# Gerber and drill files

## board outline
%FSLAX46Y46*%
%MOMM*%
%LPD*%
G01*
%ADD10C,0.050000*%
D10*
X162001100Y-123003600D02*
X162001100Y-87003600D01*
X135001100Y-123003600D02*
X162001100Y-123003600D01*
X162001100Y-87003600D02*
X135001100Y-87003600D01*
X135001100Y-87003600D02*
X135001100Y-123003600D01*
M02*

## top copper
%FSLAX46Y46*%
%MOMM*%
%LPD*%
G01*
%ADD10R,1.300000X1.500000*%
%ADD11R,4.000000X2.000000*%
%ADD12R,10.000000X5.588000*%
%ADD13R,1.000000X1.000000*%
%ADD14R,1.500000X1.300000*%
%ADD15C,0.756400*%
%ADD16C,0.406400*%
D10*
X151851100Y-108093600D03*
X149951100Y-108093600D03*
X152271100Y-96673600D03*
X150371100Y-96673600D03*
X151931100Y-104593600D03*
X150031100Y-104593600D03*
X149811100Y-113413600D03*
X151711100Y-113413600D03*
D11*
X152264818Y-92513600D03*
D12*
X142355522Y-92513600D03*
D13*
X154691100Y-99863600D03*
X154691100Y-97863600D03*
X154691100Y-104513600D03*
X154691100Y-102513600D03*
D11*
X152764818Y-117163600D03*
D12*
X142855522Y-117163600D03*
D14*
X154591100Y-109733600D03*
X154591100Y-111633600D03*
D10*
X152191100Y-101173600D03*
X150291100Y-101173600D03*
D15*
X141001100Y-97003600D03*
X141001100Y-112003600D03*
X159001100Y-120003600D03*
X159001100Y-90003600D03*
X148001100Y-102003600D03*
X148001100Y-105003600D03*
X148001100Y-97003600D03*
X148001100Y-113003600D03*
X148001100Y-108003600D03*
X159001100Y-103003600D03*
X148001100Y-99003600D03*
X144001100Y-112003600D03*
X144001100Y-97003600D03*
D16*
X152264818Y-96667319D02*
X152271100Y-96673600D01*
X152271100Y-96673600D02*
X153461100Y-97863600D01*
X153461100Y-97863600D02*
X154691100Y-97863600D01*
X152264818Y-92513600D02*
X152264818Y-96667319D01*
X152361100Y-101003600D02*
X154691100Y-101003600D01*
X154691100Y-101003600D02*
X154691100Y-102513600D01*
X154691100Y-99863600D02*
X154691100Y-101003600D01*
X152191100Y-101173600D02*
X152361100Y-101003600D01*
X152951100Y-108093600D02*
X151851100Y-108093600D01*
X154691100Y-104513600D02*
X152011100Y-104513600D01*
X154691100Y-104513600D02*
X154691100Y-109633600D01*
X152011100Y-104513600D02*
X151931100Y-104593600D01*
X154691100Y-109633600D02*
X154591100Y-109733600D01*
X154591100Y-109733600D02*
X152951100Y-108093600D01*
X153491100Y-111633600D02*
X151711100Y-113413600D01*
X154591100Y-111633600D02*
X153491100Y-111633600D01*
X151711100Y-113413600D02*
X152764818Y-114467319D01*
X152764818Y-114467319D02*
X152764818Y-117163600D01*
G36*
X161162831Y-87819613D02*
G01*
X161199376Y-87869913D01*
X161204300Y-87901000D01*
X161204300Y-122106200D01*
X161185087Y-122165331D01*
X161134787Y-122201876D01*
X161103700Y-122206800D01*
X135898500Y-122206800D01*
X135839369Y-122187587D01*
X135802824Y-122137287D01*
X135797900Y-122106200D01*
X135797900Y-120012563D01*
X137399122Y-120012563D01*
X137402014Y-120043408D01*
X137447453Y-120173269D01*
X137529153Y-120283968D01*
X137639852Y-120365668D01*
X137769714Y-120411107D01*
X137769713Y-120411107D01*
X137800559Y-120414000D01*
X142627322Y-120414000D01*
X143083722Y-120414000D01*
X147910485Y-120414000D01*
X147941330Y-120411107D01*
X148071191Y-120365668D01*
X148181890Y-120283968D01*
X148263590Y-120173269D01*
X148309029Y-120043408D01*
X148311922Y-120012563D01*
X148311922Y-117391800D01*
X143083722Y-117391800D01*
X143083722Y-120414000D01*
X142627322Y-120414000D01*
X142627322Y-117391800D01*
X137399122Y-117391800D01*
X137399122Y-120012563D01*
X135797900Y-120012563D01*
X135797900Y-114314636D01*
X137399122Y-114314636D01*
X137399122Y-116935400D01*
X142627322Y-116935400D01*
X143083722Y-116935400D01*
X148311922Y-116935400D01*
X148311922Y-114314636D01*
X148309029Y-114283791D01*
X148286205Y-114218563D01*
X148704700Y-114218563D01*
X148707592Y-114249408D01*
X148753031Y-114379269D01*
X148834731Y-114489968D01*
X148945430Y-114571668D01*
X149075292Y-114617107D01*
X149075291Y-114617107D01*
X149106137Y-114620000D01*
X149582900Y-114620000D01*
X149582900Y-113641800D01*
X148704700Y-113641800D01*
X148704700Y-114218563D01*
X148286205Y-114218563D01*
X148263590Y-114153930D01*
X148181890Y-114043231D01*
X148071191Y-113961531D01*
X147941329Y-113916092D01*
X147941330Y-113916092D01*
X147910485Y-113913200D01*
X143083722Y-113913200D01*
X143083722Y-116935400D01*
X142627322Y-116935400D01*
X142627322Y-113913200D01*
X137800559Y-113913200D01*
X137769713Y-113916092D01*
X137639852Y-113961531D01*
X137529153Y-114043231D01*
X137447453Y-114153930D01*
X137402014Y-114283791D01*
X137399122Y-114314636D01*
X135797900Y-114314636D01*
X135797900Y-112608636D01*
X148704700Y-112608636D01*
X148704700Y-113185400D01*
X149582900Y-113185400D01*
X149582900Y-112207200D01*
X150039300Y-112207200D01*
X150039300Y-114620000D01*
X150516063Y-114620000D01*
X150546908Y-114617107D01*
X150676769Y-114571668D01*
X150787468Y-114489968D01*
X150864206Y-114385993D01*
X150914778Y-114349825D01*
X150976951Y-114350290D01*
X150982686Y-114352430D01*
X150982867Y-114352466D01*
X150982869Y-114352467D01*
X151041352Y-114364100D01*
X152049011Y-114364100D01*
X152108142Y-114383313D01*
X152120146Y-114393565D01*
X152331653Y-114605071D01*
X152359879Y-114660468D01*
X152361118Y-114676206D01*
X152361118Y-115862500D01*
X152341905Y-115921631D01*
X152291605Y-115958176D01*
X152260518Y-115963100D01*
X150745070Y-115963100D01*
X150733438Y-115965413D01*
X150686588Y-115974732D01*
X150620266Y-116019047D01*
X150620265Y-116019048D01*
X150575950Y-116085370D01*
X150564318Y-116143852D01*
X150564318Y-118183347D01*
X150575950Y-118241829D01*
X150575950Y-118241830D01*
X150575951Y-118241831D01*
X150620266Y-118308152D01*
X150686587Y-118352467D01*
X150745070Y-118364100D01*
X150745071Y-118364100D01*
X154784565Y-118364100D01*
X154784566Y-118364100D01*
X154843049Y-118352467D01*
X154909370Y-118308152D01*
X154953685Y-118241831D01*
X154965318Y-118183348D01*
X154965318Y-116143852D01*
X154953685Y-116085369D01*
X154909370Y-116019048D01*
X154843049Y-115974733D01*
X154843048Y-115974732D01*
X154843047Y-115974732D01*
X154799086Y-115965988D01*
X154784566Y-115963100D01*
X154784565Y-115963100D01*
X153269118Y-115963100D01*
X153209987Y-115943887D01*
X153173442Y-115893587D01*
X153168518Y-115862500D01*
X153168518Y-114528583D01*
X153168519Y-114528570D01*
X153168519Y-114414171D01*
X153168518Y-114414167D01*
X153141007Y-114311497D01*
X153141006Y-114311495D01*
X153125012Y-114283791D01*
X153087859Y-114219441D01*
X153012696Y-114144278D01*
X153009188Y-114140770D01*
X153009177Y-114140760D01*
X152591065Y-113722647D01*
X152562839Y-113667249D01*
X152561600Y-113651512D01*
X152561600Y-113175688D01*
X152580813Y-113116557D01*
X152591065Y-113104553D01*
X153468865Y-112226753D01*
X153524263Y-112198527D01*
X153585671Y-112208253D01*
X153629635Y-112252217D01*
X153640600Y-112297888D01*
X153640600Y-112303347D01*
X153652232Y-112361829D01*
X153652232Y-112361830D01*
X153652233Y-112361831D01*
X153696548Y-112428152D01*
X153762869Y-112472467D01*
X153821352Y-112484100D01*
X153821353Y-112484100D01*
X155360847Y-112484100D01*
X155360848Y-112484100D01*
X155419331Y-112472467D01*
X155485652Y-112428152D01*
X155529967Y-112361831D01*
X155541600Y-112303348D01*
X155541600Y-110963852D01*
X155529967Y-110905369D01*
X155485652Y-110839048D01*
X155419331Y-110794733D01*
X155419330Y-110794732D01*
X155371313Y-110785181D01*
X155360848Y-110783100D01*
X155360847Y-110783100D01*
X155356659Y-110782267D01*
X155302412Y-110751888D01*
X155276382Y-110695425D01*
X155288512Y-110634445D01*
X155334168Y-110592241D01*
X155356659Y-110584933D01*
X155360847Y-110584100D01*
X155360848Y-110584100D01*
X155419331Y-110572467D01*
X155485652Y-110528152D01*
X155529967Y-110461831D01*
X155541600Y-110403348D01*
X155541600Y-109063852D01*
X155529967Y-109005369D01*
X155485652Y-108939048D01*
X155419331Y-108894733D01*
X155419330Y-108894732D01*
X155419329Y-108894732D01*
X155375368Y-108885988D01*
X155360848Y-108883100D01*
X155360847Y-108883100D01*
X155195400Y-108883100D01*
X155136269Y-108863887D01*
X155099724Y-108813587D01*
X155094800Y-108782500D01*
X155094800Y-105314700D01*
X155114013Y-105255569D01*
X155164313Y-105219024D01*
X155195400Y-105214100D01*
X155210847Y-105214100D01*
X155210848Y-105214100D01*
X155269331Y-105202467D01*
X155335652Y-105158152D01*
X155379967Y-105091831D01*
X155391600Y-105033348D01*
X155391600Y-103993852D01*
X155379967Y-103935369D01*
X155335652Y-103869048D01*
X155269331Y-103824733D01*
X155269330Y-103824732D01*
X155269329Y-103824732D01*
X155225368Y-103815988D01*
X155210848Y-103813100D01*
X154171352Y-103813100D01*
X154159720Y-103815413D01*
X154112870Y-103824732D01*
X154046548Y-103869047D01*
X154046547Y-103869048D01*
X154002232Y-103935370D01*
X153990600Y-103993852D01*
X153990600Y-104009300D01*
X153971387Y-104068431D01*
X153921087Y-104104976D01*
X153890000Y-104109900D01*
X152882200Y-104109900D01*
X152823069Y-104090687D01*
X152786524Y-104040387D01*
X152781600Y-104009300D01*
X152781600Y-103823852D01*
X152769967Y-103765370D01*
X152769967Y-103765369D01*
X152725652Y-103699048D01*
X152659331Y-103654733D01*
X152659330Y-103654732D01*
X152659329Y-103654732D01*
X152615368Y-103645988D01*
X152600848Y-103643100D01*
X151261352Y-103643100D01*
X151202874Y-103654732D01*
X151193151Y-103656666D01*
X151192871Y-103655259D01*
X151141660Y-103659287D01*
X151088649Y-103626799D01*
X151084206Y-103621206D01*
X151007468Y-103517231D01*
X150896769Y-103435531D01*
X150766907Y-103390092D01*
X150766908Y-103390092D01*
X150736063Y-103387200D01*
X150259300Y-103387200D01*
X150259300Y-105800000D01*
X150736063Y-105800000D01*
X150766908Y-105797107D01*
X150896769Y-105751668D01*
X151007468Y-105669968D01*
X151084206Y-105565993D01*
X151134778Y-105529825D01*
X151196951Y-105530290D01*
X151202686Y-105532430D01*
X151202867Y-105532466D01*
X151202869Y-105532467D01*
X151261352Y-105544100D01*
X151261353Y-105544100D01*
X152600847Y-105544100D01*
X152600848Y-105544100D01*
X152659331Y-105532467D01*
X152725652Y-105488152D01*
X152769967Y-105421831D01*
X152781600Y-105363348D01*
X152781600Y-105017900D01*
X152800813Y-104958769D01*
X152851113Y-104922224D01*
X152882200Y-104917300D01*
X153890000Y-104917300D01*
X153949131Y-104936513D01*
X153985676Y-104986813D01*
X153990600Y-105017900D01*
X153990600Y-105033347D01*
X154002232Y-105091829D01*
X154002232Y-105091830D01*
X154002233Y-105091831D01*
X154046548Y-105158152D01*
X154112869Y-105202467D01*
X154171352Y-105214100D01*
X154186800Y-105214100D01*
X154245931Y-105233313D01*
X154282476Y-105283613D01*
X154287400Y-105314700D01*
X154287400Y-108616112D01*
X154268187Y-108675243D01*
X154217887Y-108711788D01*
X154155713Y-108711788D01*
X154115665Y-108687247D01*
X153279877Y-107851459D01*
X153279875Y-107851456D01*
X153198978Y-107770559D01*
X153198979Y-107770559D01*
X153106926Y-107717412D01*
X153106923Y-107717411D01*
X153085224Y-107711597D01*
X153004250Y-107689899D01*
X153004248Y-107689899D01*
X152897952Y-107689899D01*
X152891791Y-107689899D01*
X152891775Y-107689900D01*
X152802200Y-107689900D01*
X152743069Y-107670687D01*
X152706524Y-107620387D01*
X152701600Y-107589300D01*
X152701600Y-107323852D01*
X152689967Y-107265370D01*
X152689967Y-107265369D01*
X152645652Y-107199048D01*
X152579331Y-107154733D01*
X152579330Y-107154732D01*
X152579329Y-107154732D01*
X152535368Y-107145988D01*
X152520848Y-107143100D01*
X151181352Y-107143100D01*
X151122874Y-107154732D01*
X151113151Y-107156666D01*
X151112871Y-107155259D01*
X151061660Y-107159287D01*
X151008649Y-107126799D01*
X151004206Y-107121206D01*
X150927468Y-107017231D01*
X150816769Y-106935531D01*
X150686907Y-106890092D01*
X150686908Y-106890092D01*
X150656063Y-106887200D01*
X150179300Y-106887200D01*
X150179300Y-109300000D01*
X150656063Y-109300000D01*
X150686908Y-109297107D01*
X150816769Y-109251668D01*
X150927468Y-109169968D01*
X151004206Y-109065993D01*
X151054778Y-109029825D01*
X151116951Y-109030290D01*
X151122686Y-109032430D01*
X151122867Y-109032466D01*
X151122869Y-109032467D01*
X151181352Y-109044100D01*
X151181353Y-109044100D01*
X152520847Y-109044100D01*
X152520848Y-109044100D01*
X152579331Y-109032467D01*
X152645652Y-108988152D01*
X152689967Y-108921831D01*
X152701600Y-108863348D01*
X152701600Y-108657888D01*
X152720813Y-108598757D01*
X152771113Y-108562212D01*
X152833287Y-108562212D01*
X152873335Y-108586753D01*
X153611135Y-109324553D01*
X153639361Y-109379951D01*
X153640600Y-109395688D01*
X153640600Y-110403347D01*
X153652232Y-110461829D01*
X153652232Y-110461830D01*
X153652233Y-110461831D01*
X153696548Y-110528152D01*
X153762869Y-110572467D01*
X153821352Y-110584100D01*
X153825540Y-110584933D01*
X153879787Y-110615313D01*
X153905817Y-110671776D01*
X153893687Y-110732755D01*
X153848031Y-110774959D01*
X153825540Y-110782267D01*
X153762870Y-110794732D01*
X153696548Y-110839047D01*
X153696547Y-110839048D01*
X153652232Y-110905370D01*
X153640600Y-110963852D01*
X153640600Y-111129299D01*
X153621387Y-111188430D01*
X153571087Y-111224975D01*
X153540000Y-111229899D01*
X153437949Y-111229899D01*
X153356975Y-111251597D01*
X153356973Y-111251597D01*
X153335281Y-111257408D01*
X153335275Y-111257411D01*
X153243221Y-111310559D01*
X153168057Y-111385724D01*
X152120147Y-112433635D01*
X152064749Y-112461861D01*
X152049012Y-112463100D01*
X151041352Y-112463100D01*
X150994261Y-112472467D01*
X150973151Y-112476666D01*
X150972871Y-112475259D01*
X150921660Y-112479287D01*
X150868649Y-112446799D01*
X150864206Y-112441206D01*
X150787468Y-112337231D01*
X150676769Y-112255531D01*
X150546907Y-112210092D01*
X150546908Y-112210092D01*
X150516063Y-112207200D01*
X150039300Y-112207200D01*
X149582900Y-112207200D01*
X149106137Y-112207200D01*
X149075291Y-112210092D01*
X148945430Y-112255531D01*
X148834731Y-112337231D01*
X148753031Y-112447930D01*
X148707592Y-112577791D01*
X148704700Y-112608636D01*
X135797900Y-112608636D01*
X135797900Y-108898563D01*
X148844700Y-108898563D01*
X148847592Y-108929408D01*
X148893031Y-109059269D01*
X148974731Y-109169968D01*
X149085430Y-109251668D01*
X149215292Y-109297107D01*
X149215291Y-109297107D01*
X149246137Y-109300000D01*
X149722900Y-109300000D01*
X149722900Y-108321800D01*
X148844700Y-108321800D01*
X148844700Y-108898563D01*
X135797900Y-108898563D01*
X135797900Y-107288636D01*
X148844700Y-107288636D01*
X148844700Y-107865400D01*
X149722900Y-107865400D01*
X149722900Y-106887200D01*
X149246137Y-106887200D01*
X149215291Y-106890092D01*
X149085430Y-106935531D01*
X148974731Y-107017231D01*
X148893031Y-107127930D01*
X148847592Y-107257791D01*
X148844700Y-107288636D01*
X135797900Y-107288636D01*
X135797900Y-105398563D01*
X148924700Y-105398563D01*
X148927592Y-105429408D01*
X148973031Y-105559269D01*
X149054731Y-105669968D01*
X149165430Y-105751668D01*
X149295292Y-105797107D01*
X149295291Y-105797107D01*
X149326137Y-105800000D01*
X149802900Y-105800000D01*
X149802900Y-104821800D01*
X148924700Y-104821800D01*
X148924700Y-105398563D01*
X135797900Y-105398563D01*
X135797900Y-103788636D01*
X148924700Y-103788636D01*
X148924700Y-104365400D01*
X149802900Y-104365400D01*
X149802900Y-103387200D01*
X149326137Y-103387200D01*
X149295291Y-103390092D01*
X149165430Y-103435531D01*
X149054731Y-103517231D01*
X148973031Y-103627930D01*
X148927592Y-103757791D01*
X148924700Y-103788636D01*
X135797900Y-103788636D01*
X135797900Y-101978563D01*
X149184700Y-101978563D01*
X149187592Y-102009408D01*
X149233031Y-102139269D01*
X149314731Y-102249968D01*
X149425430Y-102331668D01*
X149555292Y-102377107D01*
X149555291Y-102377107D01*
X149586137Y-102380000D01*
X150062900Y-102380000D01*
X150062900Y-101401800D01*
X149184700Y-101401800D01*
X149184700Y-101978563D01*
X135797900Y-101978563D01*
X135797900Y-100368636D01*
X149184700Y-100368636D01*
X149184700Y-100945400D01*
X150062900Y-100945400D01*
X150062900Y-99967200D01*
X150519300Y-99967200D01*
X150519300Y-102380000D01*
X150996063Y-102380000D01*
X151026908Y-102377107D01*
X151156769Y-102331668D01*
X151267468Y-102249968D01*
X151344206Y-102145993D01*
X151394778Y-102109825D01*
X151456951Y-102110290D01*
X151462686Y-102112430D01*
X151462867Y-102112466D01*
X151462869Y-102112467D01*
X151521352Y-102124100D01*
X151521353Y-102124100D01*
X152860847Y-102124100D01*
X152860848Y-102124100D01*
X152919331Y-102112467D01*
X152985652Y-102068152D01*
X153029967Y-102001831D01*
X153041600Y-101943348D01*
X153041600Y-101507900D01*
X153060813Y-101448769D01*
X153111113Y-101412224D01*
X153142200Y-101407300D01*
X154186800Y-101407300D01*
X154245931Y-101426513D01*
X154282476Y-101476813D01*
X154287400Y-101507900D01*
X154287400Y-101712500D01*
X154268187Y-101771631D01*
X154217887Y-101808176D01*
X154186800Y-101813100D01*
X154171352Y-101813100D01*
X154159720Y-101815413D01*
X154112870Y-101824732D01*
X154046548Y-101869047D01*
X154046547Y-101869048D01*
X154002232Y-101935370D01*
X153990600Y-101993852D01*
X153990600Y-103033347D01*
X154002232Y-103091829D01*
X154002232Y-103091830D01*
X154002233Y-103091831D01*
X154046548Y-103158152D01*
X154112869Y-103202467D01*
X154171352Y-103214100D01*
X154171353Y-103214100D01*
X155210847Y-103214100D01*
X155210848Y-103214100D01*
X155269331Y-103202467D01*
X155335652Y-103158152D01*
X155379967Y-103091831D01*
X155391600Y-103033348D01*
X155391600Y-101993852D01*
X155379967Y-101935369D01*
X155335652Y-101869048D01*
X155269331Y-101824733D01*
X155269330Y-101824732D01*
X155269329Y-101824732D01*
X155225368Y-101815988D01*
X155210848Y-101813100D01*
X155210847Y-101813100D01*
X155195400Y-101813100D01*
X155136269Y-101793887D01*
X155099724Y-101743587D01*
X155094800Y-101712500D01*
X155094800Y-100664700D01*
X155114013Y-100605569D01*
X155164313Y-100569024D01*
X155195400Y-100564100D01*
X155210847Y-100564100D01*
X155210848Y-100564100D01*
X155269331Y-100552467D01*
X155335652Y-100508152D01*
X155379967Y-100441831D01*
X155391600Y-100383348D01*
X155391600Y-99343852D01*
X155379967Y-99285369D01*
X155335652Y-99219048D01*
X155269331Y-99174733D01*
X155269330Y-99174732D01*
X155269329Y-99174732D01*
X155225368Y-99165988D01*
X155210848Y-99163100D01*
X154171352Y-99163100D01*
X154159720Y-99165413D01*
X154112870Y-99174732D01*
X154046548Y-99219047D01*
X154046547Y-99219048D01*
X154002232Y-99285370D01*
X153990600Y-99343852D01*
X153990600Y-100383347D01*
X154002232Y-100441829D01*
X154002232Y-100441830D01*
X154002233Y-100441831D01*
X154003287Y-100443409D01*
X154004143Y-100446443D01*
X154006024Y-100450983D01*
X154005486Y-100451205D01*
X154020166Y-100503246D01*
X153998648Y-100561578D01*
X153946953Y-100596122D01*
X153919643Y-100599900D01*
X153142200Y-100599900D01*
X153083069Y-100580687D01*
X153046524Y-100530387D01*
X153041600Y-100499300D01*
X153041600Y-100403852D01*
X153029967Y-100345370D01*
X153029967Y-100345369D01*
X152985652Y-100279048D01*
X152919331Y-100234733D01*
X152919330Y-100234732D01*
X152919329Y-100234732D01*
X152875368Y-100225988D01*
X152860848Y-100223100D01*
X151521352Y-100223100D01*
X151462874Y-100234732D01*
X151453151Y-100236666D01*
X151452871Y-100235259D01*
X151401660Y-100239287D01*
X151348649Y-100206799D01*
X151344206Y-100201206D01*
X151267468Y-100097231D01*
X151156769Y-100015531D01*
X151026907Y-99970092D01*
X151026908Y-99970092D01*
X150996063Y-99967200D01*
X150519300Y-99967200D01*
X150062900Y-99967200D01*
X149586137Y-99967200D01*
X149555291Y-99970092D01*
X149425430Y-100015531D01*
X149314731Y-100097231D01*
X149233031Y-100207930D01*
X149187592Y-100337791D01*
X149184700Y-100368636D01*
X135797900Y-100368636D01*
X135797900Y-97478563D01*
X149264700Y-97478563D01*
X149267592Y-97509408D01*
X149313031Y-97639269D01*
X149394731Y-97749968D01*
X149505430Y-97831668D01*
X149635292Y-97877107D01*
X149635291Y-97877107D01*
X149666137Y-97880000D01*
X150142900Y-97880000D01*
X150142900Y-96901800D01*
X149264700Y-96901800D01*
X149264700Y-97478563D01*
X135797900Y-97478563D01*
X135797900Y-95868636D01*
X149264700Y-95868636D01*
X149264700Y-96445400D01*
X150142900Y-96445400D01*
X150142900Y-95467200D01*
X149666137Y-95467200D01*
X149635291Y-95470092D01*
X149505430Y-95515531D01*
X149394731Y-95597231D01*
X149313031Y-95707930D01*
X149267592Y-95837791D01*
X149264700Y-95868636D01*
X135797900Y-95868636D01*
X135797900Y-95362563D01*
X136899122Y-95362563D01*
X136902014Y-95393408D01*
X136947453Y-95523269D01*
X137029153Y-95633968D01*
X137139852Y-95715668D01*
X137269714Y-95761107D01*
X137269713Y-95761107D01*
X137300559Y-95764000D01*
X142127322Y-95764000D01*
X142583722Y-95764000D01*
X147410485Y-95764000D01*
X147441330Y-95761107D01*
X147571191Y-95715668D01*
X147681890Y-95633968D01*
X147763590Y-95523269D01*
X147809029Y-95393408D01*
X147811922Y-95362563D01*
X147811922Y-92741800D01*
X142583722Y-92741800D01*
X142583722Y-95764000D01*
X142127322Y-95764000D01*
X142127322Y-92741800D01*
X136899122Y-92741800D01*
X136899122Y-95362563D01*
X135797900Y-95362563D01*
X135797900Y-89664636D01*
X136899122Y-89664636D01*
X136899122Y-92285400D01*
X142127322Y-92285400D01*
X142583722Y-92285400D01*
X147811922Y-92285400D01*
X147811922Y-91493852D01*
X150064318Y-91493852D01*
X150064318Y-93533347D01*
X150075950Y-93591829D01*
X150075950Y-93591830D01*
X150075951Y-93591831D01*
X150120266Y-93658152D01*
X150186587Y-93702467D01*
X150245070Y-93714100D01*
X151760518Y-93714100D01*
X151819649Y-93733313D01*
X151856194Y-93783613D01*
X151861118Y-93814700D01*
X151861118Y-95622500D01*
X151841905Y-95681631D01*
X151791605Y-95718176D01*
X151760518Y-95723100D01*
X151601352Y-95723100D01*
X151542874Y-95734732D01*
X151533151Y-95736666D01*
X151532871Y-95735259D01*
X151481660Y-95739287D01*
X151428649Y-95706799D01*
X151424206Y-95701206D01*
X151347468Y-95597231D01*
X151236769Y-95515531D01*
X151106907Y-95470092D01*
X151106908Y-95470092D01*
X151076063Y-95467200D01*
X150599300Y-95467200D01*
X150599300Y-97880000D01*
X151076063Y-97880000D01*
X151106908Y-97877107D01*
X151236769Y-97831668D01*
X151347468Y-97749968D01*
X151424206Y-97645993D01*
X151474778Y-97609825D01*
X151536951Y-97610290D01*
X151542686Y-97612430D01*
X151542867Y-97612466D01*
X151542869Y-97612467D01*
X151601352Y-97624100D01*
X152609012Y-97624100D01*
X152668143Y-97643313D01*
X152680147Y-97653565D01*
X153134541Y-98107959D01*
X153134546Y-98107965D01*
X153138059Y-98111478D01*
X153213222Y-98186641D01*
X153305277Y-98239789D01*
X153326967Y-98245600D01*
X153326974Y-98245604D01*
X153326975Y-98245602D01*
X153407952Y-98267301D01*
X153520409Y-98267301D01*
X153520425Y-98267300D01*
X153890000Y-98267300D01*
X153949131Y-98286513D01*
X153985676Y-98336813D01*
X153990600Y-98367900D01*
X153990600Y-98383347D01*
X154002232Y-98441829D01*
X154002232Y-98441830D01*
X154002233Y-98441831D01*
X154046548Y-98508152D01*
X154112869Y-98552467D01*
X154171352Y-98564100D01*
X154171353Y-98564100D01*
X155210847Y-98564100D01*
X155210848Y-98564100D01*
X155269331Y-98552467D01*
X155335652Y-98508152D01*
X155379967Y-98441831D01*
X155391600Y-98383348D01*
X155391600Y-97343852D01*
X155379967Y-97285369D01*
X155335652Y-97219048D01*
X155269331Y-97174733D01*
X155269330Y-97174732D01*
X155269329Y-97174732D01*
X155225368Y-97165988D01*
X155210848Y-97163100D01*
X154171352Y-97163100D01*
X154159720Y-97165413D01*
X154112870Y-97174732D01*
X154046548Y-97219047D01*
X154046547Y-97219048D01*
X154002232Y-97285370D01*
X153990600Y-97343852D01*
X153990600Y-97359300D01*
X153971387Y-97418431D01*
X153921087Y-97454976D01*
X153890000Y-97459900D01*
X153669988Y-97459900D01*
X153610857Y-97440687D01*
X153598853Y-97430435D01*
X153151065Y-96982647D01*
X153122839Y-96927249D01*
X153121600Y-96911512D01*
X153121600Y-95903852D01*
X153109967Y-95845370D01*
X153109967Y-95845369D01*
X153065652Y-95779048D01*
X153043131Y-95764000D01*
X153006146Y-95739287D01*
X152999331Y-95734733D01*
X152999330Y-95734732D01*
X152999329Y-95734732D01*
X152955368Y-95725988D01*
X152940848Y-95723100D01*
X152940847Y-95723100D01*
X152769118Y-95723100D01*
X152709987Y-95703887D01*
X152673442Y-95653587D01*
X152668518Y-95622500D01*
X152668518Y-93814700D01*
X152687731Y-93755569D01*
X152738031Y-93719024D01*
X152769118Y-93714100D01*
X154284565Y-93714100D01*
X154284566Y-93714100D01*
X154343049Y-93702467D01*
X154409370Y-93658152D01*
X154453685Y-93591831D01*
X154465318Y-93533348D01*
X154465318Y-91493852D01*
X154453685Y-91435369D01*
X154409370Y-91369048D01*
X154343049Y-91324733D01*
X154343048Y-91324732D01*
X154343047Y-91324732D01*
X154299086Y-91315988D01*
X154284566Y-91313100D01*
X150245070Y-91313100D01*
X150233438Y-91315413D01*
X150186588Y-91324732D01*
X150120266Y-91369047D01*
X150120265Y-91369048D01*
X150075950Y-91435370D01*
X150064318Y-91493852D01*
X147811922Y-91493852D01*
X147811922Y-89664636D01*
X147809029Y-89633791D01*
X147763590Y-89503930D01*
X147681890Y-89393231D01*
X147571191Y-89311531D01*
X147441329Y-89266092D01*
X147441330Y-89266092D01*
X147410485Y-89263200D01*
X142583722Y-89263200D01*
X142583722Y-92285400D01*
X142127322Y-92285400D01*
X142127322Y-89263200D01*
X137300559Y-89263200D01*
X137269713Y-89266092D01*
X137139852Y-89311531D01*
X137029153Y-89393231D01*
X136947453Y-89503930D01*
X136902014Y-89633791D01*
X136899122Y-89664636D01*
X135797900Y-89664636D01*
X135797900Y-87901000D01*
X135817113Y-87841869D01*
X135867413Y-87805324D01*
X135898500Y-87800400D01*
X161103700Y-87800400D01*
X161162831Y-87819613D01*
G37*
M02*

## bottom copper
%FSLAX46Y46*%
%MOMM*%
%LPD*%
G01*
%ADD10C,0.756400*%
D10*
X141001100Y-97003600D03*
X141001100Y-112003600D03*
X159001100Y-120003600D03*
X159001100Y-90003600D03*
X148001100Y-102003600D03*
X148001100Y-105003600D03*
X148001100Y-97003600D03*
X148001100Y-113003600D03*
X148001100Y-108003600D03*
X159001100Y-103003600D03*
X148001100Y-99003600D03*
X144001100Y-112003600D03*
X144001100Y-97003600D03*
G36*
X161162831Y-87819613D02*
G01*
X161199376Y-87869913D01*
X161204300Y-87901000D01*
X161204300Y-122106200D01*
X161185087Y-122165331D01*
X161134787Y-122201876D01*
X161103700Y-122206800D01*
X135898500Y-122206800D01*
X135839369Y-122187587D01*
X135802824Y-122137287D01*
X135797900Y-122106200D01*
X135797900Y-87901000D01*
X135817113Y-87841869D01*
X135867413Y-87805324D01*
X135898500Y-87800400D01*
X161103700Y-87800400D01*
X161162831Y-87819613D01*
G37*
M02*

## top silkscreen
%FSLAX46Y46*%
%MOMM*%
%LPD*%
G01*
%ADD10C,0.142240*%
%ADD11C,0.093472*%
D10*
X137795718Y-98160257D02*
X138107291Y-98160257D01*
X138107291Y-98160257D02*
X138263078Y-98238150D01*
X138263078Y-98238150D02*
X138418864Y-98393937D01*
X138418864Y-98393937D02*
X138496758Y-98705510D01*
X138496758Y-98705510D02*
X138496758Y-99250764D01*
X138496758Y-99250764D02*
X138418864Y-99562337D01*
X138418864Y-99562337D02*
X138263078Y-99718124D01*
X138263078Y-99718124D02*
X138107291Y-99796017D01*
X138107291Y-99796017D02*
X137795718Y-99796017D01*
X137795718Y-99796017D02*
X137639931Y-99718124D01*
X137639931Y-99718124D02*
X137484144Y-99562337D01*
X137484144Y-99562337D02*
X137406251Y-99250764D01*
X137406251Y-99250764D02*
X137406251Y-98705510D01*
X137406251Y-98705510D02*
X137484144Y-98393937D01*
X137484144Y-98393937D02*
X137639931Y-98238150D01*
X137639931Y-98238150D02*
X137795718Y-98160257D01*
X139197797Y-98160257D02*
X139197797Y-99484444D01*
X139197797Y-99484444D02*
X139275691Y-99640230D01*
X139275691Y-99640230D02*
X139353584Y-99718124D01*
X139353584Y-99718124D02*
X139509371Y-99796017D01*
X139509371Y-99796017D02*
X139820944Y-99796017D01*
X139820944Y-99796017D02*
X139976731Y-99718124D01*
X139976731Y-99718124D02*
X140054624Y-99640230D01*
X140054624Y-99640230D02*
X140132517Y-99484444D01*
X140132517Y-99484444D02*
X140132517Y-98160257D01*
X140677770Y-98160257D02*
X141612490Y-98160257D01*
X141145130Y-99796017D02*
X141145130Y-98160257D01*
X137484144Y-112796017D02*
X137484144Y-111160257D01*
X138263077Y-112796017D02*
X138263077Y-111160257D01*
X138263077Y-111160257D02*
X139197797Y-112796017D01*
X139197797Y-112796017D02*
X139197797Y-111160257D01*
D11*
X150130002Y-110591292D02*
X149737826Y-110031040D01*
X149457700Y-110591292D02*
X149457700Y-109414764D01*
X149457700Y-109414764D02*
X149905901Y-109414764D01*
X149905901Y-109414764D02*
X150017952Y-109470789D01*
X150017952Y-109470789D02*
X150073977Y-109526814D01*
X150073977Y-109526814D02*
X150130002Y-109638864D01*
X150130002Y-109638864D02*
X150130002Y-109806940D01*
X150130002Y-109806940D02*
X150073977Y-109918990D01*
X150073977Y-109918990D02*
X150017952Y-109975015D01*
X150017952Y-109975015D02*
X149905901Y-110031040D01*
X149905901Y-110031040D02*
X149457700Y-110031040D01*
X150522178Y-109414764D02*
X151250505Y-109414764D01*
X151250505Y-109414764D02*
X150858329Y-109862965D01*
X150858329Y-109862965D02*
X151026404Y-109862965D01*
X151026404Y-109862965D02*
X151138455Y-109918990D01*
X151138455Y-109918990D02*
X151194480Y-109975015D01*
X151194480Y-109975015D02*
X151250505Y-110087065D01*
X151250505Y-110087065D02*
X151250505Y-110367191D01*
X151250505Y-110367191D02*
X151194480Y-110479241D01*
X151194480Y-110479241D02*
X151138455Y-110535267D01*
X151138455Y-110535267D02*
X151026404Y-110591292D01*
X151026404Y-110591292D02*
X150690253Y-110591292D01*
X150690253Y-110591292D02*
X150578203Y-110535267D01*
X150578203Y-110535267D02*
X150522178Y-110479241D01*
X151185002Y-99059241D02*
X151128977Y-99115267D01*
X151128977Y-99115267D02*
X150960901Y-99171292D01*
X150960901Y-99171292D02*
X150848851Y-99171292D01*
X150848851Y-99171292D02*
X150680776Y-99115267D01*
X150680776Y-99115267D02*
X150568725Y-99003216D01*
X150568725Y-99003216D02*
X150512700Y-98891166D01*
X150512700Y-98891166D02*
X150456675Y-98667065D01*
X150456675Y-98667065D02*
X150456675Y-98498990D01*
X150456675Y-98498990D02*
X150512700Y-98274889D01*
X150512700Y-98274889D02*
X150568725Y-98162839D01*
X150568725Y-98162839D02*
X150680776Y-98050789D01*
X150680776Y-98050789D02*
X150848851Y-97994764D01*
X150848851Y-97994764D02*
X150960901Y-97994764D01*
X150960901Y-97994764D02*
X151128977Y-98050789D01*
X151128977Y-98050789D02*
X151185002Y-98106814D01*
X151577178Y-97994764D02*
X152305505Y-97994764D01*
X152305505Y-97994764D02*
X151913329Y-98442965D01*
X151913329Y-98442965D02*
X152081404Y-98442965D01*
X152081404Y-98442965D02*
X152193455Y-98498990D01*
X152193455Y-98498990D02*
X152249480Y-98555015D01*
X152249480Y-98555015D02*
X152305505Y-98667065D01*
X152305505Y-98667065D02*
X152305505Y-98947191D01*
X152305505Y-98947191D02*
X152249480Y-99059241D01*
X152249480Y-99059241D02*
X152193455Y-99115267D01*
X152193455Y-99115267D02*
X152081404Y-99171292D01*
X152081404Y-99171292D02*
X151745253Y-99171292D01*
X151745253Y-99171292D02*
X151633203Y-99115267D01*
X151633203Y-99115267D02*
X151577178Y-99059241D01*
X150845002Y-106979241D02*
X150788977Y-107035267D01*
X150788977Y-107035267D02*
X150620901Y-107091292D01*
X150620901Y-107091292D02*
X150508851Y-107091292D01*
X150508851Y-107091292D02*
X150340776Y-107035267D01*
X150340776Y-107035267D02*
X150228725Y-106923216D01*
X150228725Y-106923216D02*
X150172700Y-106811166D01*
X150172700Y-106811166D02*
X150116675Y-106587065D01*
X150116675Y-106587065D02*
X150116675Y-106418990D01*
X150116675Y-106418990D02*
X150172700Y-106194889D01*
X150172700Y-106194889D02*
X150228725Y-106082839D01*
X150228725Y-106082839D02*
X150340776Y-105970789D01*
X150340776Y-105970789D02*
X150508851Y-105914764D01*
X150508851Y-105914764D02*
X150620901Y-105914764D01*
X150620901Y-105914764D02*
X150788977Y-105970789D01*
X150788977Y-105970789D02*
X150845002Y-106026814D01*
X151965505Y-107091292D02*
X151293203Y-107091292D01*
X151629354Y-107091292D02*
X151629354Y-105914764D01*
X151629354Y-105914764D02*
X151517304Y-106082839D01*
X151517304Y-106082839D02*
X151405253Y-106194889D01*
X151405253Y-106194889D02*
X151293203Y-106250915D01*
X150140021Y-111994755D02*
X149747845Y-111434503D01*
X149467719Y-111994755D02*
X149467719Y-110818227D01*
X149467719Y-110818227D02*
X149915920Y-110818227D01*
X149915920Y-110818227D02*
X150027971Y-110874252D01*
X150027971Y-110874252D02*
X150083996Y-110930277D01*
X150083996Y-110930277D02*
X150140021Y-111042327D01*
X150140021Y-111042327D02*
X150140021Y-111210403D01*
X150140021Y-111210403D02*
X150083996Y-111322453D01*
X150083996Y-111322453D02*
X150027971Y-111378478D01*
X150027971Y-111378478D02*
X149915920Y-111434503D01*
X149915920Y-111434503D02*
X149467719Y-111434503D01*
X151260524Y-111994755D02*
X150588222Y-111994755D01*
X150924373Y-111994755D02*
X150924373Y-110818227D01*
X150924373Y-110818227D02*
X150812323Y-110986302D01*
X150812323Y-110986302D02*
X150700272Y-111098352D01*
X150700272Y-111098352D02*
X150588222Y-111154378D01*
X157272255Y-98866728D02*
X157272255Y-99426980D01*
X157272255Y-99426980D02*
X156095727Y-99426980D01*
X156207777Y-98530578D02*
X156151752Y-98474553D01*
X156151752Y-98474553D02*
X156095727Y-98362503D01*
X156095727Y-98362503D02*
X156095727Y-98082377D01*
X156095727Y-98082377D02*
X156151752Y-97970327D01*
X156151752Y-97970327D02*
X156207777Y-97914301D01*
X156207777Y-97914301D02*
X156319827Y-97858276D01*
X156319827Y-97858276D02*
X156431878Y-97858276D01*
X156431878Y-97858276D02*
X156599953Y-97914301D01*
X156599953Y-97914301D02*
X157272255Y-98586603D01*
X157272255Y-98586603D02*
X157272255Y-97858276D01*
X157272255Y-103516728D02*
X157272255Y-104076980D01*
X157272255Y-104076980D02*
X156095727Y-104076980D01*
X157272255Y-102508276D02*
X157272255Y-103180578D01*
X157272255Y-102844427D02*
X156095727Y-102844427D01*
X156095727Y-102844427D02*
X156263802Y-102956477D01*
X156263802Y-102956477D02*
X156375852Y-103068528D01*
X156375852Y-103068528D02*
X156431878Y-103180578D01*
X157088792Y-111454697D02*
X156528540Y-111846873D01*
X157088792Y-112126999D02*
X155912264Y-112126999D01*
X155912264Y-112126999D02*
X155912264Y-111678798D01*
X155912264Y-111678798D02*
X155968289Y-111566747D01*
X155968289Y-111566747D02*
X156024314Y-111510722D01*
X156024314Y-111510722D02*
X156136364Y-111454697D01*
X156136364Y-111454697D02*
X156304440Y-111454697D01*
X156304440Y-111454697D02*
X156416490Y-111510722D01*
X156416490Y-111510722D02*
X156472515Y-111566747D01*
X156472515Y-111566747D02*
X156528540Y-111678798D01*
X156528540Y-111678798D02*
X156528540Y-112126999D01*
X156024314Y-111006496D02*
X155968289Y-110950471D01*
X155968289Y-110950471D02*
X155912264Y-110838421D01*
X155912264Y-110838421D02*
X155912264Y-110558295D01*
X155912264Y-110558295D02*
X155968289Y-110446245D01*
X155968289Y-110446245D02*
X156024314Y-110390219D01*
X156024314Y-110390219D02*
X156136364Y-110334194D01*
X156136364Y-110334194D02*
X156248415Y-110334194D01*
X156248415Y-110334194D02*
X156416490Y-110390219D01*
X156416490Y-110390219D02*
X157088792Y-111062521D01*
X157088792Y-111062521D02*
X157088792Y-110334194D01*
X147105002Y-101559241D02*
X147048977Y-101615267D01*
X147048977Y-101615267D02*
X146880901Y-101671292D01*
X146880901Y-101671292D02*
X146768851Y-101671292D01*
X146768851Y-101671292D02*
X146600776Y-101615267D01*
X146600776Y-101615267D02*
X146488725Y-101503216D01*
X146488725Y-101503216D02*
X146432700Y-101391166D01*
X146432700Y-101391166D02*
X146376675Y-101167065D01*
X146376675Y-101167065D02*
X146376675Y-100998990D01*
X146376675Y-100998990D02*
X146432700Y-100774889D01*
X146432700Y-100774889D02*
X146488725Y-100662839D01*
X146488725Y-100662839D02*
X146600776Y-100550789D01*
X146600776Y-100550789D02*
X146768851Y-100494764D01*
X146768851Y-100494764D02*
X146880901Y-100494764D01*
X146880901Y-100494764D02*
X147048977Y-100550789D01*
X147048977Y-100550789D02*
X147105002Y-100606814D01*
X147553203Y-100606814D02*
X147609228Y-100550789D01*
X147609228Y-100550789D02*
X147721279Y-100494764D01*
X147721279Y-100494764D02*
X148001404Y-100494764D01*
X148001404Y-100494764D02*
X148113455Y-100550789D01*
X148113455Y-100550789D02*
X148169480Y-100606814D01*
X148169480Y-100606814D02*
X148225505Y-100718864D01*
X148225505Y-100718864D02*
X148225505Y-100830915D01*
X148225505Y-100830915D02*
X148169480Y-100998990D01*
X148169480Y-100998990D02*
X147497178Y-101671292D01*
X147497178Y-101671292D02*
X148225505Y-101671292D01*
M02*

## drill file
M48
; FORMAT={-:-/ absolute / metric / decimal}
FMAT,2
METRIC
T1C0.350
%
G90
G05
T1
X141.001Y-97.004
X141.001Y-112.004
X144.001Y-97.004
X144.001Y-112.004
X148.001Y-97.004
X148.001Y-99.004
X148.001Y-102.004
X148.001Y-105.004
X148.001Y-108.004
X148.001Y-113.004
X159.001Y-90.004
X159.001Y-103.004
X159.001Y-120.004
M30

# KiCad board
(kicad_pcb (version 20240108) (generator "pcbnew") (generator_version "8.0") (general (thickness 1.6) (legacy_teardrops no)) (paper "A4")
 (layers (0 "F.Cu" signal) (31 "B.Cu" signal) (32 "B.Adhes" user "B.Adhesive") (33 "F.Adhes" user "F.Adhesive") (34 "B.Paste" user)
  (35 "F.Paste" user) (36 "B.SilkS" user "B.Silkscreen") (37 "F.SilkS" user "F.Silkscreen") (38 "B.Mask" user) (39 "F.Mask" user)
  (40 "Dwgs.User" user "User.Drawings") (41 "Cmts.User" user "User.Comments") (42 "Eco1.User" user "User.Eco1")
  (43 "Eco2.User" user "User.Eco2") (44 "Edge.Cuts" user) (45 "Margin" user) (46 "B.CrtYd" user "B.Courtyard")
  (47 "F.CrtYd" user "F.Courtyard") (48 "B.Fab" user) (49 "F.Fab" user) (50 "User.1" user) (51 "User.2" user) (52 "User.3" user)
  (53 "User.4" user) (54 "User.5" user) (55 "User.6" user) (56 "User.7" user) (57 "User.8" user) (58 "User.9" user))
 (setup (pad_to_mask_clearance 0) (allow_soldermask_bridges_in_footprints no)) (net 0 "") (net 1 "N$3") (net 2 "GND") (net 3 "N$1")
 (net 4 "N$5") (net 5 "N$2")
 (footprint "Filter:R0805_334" (layer "F.Cu") (at 150.9011 108.0936 180)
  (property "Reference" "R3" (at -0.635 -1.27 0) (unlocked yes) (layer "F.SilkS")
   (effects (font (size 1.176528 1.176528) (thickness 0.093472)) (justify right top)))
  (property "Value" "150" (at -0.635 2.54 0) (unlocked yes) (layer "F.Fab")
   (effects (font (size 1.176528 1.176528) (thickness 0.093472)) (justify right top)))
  (pad "1" smd rect (at -0.95 0 180) (size 1.3 1.5) (layers "F.Cu" "F.Paste" "F.Mask") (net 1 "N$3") (solder_mask_margin 0.1016)
   (thermal_bridge_angle 0))
  (pad "2" smd rect (at 0.95 0 180) (size 1.3 1.5) (layers "F.Cu" "F.Paste" "F.Mask") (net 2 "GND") (solder_mask_margin 0.1016)
   (thermal_bridge_angle 0)))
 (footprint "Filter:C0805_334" (layer "F.Cu") (at 151.3211 96.6736 180)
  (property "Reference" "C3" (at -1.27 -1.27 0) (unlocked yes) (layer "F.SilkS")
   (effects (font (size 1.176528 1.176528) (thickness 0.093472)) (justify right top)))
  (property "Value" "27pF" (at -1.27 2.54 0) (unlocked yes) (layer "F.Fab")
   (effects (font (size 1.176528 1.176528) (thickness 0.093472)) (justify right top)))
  (pad "1" smd rect (at -0.95 0 180) (size 1.3 1.5) (layers "F.Cu" "F.Paste" "F.Mask") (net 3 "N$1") (solder_mask_margin 0.1016)
   (thermal_bridge_angle 0))
  (pad "2" smd rect (at 0.95 0 180) (size 1.3 1.5) (layers "F.Cu" "F.Paste" "F.Mask") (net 2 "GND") (solder_mask_margin 0.1016)
   (thermal_bridge_angle 0)))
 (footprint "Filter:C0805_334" (layer "F.Cu") (at 150.9811 104.5936 180)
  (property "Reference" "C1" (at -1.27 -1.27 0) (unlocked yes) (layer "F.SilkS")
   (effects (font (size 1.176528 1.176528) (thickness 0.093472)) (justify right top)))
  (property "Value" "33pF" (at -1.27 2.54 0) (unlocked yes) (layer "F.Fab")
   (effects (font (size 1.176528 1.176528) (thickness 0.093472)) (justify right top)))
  (pad "1" smd rect (at -0.95 0 180) (size 1.3 1.5) (layers "F.Cu" "F.Paste" "F.Mask") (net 1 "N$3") (solder_mask_margin 0.1016)
   (thermal_bridge_angle 0))
  (pad "2" smd rect (at 0.95 0 180) (size 1.3 1.5) (layers "F.Cu" "F.Paste" "F.Mask") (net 2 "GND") (solder_mask_margin 0.1016)
   (thermal_bridge_angle 0)))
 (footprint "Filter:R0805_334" (layer "F.Cu") (at 150.7611 113.4136)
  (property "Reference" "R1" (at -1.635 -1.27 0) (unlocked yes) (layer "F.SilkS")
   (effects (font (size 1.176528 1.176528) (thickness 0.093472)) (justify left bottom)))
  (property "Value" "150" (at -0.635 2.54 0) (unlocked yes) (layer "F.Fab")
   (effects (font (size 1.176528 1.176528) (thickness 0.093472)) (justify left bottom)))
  (pad "1" smd rect (at -0.95 0) (size 1.3 1.5) (layers "F.Cu" "F.Paste" "F.Mask") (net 2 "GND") (solder_mask_margin 0.1016)
   (thermal_bridge_angle 0))
  (pad "2" smd rect (at 0.95 0) (size 1.3 1.5) (layers "F.Cu" "F.Paste" "F.Mask") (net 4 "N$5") (solder_mask_margin 0.1016)
   (thermal_bridge_angle 0)))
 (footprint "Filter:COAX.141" (layer "F.Cu") (at 148.9011 92.5136 180)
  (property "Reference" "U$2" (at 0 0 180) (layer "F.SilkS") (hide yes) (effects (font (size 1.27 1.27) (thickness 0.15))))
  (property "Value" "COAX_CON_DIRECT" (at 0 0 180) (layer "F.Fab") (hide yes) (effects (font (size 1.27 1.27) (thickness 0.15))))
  (pad "P$1" smd rect (at -3.363718 0 180) (size 4 2) (layers "F.Cu" "F.Paste" "F.Mask") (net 3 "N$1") (solder_mask_margin 0.1016)
   (thermal_bridge_angle 0))
  (pad "P$2" smd rect (at 6.545578 0 180) (size 10 5.588) (layers "F.Cu" "F.Paste" "F.Mask") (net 2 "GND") (solder_mask_margin 0.1016)
   (thermal_bridge_angle 0)))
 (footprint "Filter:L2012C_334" (layer "F.Cu") (at 154.6911 98.8636 90)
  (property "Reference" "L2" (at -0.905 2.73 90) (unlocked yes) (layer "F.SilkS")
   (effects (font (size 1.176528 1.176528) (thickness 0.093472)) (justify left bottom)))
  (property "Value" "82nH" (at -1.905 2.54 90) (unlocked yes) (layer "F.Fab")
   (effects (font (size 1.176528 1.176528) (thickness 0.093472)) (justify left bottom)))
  (pad "1" smd rect (at -1 0 90) (size 1 1) (layers "F.Cu" "F.Paste" "F.Mask") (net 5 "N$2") (solder_mask_margin 0.1016)
   (thermal_bridge_angle 0))
  (pad "2" smd rect (at 1 0 90) (size 1 1) (layers "F.Cu" "F.Paste" "F.Mask") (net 3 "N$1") (solder_mask_margin 0.1016)
   (thermal_bridge_angle 0)))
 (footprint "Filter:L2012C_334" (layer "F.Cu") (at 154.6911 103.5136 90)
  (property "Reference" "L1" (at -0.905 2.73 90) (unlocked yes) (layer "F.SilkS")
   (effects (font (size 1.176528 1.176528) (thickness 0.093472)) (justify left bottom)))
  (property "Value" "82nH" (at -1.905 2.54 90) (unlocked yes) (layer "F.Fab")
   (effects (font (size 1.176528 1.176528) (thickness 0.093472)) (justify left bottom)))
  (pad "1" smd rect (at -1 0 90) (size 1 1) (layers "F.Cu" "F.Paste" "F.Mask") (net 1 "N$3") (solder_mask_margin 0.1016)
   (thermal_bridge_angle 0))
  (pad "2" smd rect (at 1 0 90) (size 1 1) (layers "F.Cu" "F.Paste" "F.Mask") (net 5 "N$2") (solder_mask_margin 0.1016)
   (thermal_bridge_angle 0)))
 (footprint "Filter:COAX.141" (layer "F.Cu") (at 149.4011 117.1636 180)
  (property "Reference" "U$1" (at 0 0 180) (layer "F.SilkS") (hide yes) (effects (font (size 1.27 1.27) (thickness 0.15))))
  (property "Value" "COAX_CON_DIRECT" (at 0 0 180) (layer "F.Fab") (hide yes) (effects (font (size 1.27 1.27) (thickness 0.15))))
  (pad "P$1" smd rect (at -3.363718 0 180) (size 4 2) (layers "F.Cu" "F.Paste" "F.Mask") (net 4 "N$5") (solder_mask_margin 0.1016)
   (thermal_bridge_angle 0))
  (pad "P$2" smd rect (at 6.545578 0 180) (size 10 5.588) (layers "F.Cu" "F.Paste" "F.Mask") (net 2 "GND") (solder_mask_margin 0.1016)
   (thermal_bridge_angle 0)))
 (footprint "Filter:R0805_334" (layer "F.Cu") (at 154.5911 110.6836 -90)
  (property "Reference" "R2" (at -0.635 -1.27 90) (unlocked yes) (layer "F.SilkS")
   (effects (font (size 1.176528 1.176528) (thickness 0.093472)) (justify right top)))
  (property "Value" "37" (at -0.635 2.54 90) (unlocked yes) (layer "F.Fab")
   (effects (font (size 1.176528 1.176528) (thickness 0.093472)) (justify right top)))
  (pad "1" smd rect (at -0.95 0 270) (size 1.3 1.5) (layers "F.Cu" "F.Paste" "F.Mask") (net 1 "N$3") (solder_mask_margin 0.1016)
   (thermal_bridge_angle 0))
  (pad "2" smd rect (at 0.95 0 270) (size 1.3 1.5) (layers "F.Cu" "F.Paste" "F.Mask") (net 4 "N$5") (solder_mask_margin 0.1016)
   (thermal_bridge_angle 0)))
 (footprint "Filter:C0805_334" (layer "F.Cu") (at 151.2411 101.1736 180)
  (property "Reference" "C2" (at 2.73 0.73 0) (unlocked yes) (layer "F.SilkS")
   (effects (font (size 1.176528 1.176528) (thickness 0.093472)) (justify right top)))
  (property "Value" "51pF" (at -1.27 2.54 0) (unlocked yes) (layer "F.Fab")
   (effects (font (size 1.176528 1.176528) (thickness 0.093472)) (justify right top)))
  (pad "1" smd rect (at -0.95 0 180) (size 1.3 1.5) (layers "F.Cu" "F.Paste" "F.Mask") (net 5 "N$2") (solder_mask_margin 0.1016)
   (thermal_bridge_angle 0))
  (pad "2" smd rect (at 0.95 0 180) (size 1.3 1.5) (layers "F.Cu" "F.Paste" "F.Mask") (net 2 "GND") (solder_mask_margin 0.1016)
   (thermal_bridge_angle 0)))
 (gr_line (start 162.0011 123.0036) (end 162.0011 87.0036) (stroke (width 0.05) (type solid)) (layer "Edge.Cuts"))
 (gr_line (start 135.0011 123.0036) (end 162.0011 123.0036) (stroke (width 0.05) (type solid)) (layer "Edge.Cuts"))
 (gr_line (start 162.0011 87.0036) (end 135.0011 87.0036) (stroke (width 0.05) (type solid)) (layer "Edge.Cuts"))
 (gr_line (start 135.0011 87.0036) (end 135.0011 123.0036) (stroke (width 0.05) (type solid)) (layer "Edge.Cuts"))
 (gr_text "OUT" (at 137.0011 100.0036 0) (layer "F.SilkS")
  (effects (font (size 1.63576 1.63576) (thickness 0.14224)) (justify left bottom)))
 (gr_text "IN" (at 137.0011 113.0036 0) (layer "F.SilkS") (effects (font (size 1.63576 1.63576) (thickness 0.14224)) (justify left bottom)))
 (via (at 141.0011 97.0036) (size 0.7564) (drill 0.35) (layers "F.Cu" "B.Cu") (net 2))
 (via (at 141.0011 112.0036) (size 0.7564) (drill 0.35) (layers "F.Cu" "B.Cu") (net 2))
 (via (at 159.0011 120.0036) (size 0.7564) (drill 0.35) (layers "F.Cu" "B.Cu") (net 2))
 (via (at 159.0011 90.0036) (size 0.7564) (drill 0.35) (layers "F.Cu" "B.Cu") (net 2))
 (via (at 148.0011 102.0036) (size 0.7564) (drill 0.35) (layers "F.Cu" "B.Cu") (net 2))
 (via (at 148.0011 105.0036) (size 0.7564) (drill 0.35) (layers "F.Cu" "B.Cu") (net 2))
 (via (at 148.0011 97.0036) (size 0.7564) (drill 0.35) (layers "F.Cu" "B.Cu") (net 2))
 (via (at 148.0011 113.0036) (size 0.7564) (drill 0.35) (layers "F.Cu" "B.Cu") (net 2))
 (via (at 148.0011 108.0036) (size 0.7564) (drill 0.35) (layers "F.Cu" "B.Cu") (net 2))
 (via (at 159.0011 103.0036) (size 0.7564) (drill 0.35) (layers "F.Cu" "B.Cu") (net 2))
 (via (at 148.0011 99.0036) (size 0.7564) (drill 0.35) (layers "F.Cu" "B.Cu") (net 2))
 (via (at 144.0011 112.0036) (size 0.7564) (drill 0.35) (layers "F.Cu" "B.Cu") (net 2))
 (via (at 144.0011 97.0036) (size 0.7564) (drill 0.35) (layers "F.Cu" "B.Cu") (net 2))
 (segment (start 152.264818 96.667319) (end 152.2711 96.6736) (width 0.4064) (layer "F.Cu") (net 3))
 (segment (start 152.2711 96.6736) (end 153.4611 97.8636) (width 0.4064) (layer "F.Cu") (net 3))
 (segment (start 153.4611 97.8636) (end 154.6911 97.8636) (width 0.4064) (layer "F.Cu") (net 3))
 (segment (start 152.264818 92.5136) (end 152.264818 96.667319) (width 0.4064) (layer "F.Cu") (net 3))
 (segment (start 152.3611 101.0036) (end 154.6911 101.0036) (width 0.4064) (layer "F.Cu") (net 5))
 (segment (start 154.6911 101.0036) (end 154.6911 102.5136) (width 0.4064) (layer "F.Cu") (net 5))
 (segment (start 154.6911 99.8636) (end 154.6911 101.0036) (width 0.4064) (layer "F.Cu") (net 5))
 (segment (start 152.1911 101.1736) (end 152.3611 101.0036) (width 0.4064) (layer "F.Cu") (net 5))
 (segment (start 152.9511 108.0936) (end 151.8511 108.0936) (width 0.4064) (layer "F.Cu") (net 1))
 (segment (start 154.6911 104.5136) (end 152.0111 104.5136) (width 0.4064) (layer "F.Cu") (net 1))
 (segment (start 154.6911 104.5136) (end 154.6911 109.6336) (width 0.4064) (layer "F.Cu") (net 1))
 (segment (start 152.0111 104.5136) (end 151.9311 104.5936) (width 0.4064) (layer "F.Cu") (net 1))
 (segment (start 154.6911 109.6336) (end 154.5911 109.7336) (width 0.4064) (layer "F.Cu") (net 1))
 (segment (start 154.5911 109.7336) (end 152.9511 108.0936) (width 0.4064) (layer "F.Cu") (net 1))
 (segment (start 153.4911 111.6336) (end 151.7111 113.4136) (width 0.4064) (layer "F.Cu") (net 4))
 (segment (start 154.5911 111.6336) (end 153.4911 111.6336) (width 0.4064) (layer "F.Cu") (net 4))
 (segment (start 151.7111 113.4136) (end 152.764818 114.467319) (width 0.4064) (layer "F.Cu") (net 4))
 (segment (start 152.764818 114.467319) (end 152.764818 117.1636) (width 0.4064) (layer "F.Cu") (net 4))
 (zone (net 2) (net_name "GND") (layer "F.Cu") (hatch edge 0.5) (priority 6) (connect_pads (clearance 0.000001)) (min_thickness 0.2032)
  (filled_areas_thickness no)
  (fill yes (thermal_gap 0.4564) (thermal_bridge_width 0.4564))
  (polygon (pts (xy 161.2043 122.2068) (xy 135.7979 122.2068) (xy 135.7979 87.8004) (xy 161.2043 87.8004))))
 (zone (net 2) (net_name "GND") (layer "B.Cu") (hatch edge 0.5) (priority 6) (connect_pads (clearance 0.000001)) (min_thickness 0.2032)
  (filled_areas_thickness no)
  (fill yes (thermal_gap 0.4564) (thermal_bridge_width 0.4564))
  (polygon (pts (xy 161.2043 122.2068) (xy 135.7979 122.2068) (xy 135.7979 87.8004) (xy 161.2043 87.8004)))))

